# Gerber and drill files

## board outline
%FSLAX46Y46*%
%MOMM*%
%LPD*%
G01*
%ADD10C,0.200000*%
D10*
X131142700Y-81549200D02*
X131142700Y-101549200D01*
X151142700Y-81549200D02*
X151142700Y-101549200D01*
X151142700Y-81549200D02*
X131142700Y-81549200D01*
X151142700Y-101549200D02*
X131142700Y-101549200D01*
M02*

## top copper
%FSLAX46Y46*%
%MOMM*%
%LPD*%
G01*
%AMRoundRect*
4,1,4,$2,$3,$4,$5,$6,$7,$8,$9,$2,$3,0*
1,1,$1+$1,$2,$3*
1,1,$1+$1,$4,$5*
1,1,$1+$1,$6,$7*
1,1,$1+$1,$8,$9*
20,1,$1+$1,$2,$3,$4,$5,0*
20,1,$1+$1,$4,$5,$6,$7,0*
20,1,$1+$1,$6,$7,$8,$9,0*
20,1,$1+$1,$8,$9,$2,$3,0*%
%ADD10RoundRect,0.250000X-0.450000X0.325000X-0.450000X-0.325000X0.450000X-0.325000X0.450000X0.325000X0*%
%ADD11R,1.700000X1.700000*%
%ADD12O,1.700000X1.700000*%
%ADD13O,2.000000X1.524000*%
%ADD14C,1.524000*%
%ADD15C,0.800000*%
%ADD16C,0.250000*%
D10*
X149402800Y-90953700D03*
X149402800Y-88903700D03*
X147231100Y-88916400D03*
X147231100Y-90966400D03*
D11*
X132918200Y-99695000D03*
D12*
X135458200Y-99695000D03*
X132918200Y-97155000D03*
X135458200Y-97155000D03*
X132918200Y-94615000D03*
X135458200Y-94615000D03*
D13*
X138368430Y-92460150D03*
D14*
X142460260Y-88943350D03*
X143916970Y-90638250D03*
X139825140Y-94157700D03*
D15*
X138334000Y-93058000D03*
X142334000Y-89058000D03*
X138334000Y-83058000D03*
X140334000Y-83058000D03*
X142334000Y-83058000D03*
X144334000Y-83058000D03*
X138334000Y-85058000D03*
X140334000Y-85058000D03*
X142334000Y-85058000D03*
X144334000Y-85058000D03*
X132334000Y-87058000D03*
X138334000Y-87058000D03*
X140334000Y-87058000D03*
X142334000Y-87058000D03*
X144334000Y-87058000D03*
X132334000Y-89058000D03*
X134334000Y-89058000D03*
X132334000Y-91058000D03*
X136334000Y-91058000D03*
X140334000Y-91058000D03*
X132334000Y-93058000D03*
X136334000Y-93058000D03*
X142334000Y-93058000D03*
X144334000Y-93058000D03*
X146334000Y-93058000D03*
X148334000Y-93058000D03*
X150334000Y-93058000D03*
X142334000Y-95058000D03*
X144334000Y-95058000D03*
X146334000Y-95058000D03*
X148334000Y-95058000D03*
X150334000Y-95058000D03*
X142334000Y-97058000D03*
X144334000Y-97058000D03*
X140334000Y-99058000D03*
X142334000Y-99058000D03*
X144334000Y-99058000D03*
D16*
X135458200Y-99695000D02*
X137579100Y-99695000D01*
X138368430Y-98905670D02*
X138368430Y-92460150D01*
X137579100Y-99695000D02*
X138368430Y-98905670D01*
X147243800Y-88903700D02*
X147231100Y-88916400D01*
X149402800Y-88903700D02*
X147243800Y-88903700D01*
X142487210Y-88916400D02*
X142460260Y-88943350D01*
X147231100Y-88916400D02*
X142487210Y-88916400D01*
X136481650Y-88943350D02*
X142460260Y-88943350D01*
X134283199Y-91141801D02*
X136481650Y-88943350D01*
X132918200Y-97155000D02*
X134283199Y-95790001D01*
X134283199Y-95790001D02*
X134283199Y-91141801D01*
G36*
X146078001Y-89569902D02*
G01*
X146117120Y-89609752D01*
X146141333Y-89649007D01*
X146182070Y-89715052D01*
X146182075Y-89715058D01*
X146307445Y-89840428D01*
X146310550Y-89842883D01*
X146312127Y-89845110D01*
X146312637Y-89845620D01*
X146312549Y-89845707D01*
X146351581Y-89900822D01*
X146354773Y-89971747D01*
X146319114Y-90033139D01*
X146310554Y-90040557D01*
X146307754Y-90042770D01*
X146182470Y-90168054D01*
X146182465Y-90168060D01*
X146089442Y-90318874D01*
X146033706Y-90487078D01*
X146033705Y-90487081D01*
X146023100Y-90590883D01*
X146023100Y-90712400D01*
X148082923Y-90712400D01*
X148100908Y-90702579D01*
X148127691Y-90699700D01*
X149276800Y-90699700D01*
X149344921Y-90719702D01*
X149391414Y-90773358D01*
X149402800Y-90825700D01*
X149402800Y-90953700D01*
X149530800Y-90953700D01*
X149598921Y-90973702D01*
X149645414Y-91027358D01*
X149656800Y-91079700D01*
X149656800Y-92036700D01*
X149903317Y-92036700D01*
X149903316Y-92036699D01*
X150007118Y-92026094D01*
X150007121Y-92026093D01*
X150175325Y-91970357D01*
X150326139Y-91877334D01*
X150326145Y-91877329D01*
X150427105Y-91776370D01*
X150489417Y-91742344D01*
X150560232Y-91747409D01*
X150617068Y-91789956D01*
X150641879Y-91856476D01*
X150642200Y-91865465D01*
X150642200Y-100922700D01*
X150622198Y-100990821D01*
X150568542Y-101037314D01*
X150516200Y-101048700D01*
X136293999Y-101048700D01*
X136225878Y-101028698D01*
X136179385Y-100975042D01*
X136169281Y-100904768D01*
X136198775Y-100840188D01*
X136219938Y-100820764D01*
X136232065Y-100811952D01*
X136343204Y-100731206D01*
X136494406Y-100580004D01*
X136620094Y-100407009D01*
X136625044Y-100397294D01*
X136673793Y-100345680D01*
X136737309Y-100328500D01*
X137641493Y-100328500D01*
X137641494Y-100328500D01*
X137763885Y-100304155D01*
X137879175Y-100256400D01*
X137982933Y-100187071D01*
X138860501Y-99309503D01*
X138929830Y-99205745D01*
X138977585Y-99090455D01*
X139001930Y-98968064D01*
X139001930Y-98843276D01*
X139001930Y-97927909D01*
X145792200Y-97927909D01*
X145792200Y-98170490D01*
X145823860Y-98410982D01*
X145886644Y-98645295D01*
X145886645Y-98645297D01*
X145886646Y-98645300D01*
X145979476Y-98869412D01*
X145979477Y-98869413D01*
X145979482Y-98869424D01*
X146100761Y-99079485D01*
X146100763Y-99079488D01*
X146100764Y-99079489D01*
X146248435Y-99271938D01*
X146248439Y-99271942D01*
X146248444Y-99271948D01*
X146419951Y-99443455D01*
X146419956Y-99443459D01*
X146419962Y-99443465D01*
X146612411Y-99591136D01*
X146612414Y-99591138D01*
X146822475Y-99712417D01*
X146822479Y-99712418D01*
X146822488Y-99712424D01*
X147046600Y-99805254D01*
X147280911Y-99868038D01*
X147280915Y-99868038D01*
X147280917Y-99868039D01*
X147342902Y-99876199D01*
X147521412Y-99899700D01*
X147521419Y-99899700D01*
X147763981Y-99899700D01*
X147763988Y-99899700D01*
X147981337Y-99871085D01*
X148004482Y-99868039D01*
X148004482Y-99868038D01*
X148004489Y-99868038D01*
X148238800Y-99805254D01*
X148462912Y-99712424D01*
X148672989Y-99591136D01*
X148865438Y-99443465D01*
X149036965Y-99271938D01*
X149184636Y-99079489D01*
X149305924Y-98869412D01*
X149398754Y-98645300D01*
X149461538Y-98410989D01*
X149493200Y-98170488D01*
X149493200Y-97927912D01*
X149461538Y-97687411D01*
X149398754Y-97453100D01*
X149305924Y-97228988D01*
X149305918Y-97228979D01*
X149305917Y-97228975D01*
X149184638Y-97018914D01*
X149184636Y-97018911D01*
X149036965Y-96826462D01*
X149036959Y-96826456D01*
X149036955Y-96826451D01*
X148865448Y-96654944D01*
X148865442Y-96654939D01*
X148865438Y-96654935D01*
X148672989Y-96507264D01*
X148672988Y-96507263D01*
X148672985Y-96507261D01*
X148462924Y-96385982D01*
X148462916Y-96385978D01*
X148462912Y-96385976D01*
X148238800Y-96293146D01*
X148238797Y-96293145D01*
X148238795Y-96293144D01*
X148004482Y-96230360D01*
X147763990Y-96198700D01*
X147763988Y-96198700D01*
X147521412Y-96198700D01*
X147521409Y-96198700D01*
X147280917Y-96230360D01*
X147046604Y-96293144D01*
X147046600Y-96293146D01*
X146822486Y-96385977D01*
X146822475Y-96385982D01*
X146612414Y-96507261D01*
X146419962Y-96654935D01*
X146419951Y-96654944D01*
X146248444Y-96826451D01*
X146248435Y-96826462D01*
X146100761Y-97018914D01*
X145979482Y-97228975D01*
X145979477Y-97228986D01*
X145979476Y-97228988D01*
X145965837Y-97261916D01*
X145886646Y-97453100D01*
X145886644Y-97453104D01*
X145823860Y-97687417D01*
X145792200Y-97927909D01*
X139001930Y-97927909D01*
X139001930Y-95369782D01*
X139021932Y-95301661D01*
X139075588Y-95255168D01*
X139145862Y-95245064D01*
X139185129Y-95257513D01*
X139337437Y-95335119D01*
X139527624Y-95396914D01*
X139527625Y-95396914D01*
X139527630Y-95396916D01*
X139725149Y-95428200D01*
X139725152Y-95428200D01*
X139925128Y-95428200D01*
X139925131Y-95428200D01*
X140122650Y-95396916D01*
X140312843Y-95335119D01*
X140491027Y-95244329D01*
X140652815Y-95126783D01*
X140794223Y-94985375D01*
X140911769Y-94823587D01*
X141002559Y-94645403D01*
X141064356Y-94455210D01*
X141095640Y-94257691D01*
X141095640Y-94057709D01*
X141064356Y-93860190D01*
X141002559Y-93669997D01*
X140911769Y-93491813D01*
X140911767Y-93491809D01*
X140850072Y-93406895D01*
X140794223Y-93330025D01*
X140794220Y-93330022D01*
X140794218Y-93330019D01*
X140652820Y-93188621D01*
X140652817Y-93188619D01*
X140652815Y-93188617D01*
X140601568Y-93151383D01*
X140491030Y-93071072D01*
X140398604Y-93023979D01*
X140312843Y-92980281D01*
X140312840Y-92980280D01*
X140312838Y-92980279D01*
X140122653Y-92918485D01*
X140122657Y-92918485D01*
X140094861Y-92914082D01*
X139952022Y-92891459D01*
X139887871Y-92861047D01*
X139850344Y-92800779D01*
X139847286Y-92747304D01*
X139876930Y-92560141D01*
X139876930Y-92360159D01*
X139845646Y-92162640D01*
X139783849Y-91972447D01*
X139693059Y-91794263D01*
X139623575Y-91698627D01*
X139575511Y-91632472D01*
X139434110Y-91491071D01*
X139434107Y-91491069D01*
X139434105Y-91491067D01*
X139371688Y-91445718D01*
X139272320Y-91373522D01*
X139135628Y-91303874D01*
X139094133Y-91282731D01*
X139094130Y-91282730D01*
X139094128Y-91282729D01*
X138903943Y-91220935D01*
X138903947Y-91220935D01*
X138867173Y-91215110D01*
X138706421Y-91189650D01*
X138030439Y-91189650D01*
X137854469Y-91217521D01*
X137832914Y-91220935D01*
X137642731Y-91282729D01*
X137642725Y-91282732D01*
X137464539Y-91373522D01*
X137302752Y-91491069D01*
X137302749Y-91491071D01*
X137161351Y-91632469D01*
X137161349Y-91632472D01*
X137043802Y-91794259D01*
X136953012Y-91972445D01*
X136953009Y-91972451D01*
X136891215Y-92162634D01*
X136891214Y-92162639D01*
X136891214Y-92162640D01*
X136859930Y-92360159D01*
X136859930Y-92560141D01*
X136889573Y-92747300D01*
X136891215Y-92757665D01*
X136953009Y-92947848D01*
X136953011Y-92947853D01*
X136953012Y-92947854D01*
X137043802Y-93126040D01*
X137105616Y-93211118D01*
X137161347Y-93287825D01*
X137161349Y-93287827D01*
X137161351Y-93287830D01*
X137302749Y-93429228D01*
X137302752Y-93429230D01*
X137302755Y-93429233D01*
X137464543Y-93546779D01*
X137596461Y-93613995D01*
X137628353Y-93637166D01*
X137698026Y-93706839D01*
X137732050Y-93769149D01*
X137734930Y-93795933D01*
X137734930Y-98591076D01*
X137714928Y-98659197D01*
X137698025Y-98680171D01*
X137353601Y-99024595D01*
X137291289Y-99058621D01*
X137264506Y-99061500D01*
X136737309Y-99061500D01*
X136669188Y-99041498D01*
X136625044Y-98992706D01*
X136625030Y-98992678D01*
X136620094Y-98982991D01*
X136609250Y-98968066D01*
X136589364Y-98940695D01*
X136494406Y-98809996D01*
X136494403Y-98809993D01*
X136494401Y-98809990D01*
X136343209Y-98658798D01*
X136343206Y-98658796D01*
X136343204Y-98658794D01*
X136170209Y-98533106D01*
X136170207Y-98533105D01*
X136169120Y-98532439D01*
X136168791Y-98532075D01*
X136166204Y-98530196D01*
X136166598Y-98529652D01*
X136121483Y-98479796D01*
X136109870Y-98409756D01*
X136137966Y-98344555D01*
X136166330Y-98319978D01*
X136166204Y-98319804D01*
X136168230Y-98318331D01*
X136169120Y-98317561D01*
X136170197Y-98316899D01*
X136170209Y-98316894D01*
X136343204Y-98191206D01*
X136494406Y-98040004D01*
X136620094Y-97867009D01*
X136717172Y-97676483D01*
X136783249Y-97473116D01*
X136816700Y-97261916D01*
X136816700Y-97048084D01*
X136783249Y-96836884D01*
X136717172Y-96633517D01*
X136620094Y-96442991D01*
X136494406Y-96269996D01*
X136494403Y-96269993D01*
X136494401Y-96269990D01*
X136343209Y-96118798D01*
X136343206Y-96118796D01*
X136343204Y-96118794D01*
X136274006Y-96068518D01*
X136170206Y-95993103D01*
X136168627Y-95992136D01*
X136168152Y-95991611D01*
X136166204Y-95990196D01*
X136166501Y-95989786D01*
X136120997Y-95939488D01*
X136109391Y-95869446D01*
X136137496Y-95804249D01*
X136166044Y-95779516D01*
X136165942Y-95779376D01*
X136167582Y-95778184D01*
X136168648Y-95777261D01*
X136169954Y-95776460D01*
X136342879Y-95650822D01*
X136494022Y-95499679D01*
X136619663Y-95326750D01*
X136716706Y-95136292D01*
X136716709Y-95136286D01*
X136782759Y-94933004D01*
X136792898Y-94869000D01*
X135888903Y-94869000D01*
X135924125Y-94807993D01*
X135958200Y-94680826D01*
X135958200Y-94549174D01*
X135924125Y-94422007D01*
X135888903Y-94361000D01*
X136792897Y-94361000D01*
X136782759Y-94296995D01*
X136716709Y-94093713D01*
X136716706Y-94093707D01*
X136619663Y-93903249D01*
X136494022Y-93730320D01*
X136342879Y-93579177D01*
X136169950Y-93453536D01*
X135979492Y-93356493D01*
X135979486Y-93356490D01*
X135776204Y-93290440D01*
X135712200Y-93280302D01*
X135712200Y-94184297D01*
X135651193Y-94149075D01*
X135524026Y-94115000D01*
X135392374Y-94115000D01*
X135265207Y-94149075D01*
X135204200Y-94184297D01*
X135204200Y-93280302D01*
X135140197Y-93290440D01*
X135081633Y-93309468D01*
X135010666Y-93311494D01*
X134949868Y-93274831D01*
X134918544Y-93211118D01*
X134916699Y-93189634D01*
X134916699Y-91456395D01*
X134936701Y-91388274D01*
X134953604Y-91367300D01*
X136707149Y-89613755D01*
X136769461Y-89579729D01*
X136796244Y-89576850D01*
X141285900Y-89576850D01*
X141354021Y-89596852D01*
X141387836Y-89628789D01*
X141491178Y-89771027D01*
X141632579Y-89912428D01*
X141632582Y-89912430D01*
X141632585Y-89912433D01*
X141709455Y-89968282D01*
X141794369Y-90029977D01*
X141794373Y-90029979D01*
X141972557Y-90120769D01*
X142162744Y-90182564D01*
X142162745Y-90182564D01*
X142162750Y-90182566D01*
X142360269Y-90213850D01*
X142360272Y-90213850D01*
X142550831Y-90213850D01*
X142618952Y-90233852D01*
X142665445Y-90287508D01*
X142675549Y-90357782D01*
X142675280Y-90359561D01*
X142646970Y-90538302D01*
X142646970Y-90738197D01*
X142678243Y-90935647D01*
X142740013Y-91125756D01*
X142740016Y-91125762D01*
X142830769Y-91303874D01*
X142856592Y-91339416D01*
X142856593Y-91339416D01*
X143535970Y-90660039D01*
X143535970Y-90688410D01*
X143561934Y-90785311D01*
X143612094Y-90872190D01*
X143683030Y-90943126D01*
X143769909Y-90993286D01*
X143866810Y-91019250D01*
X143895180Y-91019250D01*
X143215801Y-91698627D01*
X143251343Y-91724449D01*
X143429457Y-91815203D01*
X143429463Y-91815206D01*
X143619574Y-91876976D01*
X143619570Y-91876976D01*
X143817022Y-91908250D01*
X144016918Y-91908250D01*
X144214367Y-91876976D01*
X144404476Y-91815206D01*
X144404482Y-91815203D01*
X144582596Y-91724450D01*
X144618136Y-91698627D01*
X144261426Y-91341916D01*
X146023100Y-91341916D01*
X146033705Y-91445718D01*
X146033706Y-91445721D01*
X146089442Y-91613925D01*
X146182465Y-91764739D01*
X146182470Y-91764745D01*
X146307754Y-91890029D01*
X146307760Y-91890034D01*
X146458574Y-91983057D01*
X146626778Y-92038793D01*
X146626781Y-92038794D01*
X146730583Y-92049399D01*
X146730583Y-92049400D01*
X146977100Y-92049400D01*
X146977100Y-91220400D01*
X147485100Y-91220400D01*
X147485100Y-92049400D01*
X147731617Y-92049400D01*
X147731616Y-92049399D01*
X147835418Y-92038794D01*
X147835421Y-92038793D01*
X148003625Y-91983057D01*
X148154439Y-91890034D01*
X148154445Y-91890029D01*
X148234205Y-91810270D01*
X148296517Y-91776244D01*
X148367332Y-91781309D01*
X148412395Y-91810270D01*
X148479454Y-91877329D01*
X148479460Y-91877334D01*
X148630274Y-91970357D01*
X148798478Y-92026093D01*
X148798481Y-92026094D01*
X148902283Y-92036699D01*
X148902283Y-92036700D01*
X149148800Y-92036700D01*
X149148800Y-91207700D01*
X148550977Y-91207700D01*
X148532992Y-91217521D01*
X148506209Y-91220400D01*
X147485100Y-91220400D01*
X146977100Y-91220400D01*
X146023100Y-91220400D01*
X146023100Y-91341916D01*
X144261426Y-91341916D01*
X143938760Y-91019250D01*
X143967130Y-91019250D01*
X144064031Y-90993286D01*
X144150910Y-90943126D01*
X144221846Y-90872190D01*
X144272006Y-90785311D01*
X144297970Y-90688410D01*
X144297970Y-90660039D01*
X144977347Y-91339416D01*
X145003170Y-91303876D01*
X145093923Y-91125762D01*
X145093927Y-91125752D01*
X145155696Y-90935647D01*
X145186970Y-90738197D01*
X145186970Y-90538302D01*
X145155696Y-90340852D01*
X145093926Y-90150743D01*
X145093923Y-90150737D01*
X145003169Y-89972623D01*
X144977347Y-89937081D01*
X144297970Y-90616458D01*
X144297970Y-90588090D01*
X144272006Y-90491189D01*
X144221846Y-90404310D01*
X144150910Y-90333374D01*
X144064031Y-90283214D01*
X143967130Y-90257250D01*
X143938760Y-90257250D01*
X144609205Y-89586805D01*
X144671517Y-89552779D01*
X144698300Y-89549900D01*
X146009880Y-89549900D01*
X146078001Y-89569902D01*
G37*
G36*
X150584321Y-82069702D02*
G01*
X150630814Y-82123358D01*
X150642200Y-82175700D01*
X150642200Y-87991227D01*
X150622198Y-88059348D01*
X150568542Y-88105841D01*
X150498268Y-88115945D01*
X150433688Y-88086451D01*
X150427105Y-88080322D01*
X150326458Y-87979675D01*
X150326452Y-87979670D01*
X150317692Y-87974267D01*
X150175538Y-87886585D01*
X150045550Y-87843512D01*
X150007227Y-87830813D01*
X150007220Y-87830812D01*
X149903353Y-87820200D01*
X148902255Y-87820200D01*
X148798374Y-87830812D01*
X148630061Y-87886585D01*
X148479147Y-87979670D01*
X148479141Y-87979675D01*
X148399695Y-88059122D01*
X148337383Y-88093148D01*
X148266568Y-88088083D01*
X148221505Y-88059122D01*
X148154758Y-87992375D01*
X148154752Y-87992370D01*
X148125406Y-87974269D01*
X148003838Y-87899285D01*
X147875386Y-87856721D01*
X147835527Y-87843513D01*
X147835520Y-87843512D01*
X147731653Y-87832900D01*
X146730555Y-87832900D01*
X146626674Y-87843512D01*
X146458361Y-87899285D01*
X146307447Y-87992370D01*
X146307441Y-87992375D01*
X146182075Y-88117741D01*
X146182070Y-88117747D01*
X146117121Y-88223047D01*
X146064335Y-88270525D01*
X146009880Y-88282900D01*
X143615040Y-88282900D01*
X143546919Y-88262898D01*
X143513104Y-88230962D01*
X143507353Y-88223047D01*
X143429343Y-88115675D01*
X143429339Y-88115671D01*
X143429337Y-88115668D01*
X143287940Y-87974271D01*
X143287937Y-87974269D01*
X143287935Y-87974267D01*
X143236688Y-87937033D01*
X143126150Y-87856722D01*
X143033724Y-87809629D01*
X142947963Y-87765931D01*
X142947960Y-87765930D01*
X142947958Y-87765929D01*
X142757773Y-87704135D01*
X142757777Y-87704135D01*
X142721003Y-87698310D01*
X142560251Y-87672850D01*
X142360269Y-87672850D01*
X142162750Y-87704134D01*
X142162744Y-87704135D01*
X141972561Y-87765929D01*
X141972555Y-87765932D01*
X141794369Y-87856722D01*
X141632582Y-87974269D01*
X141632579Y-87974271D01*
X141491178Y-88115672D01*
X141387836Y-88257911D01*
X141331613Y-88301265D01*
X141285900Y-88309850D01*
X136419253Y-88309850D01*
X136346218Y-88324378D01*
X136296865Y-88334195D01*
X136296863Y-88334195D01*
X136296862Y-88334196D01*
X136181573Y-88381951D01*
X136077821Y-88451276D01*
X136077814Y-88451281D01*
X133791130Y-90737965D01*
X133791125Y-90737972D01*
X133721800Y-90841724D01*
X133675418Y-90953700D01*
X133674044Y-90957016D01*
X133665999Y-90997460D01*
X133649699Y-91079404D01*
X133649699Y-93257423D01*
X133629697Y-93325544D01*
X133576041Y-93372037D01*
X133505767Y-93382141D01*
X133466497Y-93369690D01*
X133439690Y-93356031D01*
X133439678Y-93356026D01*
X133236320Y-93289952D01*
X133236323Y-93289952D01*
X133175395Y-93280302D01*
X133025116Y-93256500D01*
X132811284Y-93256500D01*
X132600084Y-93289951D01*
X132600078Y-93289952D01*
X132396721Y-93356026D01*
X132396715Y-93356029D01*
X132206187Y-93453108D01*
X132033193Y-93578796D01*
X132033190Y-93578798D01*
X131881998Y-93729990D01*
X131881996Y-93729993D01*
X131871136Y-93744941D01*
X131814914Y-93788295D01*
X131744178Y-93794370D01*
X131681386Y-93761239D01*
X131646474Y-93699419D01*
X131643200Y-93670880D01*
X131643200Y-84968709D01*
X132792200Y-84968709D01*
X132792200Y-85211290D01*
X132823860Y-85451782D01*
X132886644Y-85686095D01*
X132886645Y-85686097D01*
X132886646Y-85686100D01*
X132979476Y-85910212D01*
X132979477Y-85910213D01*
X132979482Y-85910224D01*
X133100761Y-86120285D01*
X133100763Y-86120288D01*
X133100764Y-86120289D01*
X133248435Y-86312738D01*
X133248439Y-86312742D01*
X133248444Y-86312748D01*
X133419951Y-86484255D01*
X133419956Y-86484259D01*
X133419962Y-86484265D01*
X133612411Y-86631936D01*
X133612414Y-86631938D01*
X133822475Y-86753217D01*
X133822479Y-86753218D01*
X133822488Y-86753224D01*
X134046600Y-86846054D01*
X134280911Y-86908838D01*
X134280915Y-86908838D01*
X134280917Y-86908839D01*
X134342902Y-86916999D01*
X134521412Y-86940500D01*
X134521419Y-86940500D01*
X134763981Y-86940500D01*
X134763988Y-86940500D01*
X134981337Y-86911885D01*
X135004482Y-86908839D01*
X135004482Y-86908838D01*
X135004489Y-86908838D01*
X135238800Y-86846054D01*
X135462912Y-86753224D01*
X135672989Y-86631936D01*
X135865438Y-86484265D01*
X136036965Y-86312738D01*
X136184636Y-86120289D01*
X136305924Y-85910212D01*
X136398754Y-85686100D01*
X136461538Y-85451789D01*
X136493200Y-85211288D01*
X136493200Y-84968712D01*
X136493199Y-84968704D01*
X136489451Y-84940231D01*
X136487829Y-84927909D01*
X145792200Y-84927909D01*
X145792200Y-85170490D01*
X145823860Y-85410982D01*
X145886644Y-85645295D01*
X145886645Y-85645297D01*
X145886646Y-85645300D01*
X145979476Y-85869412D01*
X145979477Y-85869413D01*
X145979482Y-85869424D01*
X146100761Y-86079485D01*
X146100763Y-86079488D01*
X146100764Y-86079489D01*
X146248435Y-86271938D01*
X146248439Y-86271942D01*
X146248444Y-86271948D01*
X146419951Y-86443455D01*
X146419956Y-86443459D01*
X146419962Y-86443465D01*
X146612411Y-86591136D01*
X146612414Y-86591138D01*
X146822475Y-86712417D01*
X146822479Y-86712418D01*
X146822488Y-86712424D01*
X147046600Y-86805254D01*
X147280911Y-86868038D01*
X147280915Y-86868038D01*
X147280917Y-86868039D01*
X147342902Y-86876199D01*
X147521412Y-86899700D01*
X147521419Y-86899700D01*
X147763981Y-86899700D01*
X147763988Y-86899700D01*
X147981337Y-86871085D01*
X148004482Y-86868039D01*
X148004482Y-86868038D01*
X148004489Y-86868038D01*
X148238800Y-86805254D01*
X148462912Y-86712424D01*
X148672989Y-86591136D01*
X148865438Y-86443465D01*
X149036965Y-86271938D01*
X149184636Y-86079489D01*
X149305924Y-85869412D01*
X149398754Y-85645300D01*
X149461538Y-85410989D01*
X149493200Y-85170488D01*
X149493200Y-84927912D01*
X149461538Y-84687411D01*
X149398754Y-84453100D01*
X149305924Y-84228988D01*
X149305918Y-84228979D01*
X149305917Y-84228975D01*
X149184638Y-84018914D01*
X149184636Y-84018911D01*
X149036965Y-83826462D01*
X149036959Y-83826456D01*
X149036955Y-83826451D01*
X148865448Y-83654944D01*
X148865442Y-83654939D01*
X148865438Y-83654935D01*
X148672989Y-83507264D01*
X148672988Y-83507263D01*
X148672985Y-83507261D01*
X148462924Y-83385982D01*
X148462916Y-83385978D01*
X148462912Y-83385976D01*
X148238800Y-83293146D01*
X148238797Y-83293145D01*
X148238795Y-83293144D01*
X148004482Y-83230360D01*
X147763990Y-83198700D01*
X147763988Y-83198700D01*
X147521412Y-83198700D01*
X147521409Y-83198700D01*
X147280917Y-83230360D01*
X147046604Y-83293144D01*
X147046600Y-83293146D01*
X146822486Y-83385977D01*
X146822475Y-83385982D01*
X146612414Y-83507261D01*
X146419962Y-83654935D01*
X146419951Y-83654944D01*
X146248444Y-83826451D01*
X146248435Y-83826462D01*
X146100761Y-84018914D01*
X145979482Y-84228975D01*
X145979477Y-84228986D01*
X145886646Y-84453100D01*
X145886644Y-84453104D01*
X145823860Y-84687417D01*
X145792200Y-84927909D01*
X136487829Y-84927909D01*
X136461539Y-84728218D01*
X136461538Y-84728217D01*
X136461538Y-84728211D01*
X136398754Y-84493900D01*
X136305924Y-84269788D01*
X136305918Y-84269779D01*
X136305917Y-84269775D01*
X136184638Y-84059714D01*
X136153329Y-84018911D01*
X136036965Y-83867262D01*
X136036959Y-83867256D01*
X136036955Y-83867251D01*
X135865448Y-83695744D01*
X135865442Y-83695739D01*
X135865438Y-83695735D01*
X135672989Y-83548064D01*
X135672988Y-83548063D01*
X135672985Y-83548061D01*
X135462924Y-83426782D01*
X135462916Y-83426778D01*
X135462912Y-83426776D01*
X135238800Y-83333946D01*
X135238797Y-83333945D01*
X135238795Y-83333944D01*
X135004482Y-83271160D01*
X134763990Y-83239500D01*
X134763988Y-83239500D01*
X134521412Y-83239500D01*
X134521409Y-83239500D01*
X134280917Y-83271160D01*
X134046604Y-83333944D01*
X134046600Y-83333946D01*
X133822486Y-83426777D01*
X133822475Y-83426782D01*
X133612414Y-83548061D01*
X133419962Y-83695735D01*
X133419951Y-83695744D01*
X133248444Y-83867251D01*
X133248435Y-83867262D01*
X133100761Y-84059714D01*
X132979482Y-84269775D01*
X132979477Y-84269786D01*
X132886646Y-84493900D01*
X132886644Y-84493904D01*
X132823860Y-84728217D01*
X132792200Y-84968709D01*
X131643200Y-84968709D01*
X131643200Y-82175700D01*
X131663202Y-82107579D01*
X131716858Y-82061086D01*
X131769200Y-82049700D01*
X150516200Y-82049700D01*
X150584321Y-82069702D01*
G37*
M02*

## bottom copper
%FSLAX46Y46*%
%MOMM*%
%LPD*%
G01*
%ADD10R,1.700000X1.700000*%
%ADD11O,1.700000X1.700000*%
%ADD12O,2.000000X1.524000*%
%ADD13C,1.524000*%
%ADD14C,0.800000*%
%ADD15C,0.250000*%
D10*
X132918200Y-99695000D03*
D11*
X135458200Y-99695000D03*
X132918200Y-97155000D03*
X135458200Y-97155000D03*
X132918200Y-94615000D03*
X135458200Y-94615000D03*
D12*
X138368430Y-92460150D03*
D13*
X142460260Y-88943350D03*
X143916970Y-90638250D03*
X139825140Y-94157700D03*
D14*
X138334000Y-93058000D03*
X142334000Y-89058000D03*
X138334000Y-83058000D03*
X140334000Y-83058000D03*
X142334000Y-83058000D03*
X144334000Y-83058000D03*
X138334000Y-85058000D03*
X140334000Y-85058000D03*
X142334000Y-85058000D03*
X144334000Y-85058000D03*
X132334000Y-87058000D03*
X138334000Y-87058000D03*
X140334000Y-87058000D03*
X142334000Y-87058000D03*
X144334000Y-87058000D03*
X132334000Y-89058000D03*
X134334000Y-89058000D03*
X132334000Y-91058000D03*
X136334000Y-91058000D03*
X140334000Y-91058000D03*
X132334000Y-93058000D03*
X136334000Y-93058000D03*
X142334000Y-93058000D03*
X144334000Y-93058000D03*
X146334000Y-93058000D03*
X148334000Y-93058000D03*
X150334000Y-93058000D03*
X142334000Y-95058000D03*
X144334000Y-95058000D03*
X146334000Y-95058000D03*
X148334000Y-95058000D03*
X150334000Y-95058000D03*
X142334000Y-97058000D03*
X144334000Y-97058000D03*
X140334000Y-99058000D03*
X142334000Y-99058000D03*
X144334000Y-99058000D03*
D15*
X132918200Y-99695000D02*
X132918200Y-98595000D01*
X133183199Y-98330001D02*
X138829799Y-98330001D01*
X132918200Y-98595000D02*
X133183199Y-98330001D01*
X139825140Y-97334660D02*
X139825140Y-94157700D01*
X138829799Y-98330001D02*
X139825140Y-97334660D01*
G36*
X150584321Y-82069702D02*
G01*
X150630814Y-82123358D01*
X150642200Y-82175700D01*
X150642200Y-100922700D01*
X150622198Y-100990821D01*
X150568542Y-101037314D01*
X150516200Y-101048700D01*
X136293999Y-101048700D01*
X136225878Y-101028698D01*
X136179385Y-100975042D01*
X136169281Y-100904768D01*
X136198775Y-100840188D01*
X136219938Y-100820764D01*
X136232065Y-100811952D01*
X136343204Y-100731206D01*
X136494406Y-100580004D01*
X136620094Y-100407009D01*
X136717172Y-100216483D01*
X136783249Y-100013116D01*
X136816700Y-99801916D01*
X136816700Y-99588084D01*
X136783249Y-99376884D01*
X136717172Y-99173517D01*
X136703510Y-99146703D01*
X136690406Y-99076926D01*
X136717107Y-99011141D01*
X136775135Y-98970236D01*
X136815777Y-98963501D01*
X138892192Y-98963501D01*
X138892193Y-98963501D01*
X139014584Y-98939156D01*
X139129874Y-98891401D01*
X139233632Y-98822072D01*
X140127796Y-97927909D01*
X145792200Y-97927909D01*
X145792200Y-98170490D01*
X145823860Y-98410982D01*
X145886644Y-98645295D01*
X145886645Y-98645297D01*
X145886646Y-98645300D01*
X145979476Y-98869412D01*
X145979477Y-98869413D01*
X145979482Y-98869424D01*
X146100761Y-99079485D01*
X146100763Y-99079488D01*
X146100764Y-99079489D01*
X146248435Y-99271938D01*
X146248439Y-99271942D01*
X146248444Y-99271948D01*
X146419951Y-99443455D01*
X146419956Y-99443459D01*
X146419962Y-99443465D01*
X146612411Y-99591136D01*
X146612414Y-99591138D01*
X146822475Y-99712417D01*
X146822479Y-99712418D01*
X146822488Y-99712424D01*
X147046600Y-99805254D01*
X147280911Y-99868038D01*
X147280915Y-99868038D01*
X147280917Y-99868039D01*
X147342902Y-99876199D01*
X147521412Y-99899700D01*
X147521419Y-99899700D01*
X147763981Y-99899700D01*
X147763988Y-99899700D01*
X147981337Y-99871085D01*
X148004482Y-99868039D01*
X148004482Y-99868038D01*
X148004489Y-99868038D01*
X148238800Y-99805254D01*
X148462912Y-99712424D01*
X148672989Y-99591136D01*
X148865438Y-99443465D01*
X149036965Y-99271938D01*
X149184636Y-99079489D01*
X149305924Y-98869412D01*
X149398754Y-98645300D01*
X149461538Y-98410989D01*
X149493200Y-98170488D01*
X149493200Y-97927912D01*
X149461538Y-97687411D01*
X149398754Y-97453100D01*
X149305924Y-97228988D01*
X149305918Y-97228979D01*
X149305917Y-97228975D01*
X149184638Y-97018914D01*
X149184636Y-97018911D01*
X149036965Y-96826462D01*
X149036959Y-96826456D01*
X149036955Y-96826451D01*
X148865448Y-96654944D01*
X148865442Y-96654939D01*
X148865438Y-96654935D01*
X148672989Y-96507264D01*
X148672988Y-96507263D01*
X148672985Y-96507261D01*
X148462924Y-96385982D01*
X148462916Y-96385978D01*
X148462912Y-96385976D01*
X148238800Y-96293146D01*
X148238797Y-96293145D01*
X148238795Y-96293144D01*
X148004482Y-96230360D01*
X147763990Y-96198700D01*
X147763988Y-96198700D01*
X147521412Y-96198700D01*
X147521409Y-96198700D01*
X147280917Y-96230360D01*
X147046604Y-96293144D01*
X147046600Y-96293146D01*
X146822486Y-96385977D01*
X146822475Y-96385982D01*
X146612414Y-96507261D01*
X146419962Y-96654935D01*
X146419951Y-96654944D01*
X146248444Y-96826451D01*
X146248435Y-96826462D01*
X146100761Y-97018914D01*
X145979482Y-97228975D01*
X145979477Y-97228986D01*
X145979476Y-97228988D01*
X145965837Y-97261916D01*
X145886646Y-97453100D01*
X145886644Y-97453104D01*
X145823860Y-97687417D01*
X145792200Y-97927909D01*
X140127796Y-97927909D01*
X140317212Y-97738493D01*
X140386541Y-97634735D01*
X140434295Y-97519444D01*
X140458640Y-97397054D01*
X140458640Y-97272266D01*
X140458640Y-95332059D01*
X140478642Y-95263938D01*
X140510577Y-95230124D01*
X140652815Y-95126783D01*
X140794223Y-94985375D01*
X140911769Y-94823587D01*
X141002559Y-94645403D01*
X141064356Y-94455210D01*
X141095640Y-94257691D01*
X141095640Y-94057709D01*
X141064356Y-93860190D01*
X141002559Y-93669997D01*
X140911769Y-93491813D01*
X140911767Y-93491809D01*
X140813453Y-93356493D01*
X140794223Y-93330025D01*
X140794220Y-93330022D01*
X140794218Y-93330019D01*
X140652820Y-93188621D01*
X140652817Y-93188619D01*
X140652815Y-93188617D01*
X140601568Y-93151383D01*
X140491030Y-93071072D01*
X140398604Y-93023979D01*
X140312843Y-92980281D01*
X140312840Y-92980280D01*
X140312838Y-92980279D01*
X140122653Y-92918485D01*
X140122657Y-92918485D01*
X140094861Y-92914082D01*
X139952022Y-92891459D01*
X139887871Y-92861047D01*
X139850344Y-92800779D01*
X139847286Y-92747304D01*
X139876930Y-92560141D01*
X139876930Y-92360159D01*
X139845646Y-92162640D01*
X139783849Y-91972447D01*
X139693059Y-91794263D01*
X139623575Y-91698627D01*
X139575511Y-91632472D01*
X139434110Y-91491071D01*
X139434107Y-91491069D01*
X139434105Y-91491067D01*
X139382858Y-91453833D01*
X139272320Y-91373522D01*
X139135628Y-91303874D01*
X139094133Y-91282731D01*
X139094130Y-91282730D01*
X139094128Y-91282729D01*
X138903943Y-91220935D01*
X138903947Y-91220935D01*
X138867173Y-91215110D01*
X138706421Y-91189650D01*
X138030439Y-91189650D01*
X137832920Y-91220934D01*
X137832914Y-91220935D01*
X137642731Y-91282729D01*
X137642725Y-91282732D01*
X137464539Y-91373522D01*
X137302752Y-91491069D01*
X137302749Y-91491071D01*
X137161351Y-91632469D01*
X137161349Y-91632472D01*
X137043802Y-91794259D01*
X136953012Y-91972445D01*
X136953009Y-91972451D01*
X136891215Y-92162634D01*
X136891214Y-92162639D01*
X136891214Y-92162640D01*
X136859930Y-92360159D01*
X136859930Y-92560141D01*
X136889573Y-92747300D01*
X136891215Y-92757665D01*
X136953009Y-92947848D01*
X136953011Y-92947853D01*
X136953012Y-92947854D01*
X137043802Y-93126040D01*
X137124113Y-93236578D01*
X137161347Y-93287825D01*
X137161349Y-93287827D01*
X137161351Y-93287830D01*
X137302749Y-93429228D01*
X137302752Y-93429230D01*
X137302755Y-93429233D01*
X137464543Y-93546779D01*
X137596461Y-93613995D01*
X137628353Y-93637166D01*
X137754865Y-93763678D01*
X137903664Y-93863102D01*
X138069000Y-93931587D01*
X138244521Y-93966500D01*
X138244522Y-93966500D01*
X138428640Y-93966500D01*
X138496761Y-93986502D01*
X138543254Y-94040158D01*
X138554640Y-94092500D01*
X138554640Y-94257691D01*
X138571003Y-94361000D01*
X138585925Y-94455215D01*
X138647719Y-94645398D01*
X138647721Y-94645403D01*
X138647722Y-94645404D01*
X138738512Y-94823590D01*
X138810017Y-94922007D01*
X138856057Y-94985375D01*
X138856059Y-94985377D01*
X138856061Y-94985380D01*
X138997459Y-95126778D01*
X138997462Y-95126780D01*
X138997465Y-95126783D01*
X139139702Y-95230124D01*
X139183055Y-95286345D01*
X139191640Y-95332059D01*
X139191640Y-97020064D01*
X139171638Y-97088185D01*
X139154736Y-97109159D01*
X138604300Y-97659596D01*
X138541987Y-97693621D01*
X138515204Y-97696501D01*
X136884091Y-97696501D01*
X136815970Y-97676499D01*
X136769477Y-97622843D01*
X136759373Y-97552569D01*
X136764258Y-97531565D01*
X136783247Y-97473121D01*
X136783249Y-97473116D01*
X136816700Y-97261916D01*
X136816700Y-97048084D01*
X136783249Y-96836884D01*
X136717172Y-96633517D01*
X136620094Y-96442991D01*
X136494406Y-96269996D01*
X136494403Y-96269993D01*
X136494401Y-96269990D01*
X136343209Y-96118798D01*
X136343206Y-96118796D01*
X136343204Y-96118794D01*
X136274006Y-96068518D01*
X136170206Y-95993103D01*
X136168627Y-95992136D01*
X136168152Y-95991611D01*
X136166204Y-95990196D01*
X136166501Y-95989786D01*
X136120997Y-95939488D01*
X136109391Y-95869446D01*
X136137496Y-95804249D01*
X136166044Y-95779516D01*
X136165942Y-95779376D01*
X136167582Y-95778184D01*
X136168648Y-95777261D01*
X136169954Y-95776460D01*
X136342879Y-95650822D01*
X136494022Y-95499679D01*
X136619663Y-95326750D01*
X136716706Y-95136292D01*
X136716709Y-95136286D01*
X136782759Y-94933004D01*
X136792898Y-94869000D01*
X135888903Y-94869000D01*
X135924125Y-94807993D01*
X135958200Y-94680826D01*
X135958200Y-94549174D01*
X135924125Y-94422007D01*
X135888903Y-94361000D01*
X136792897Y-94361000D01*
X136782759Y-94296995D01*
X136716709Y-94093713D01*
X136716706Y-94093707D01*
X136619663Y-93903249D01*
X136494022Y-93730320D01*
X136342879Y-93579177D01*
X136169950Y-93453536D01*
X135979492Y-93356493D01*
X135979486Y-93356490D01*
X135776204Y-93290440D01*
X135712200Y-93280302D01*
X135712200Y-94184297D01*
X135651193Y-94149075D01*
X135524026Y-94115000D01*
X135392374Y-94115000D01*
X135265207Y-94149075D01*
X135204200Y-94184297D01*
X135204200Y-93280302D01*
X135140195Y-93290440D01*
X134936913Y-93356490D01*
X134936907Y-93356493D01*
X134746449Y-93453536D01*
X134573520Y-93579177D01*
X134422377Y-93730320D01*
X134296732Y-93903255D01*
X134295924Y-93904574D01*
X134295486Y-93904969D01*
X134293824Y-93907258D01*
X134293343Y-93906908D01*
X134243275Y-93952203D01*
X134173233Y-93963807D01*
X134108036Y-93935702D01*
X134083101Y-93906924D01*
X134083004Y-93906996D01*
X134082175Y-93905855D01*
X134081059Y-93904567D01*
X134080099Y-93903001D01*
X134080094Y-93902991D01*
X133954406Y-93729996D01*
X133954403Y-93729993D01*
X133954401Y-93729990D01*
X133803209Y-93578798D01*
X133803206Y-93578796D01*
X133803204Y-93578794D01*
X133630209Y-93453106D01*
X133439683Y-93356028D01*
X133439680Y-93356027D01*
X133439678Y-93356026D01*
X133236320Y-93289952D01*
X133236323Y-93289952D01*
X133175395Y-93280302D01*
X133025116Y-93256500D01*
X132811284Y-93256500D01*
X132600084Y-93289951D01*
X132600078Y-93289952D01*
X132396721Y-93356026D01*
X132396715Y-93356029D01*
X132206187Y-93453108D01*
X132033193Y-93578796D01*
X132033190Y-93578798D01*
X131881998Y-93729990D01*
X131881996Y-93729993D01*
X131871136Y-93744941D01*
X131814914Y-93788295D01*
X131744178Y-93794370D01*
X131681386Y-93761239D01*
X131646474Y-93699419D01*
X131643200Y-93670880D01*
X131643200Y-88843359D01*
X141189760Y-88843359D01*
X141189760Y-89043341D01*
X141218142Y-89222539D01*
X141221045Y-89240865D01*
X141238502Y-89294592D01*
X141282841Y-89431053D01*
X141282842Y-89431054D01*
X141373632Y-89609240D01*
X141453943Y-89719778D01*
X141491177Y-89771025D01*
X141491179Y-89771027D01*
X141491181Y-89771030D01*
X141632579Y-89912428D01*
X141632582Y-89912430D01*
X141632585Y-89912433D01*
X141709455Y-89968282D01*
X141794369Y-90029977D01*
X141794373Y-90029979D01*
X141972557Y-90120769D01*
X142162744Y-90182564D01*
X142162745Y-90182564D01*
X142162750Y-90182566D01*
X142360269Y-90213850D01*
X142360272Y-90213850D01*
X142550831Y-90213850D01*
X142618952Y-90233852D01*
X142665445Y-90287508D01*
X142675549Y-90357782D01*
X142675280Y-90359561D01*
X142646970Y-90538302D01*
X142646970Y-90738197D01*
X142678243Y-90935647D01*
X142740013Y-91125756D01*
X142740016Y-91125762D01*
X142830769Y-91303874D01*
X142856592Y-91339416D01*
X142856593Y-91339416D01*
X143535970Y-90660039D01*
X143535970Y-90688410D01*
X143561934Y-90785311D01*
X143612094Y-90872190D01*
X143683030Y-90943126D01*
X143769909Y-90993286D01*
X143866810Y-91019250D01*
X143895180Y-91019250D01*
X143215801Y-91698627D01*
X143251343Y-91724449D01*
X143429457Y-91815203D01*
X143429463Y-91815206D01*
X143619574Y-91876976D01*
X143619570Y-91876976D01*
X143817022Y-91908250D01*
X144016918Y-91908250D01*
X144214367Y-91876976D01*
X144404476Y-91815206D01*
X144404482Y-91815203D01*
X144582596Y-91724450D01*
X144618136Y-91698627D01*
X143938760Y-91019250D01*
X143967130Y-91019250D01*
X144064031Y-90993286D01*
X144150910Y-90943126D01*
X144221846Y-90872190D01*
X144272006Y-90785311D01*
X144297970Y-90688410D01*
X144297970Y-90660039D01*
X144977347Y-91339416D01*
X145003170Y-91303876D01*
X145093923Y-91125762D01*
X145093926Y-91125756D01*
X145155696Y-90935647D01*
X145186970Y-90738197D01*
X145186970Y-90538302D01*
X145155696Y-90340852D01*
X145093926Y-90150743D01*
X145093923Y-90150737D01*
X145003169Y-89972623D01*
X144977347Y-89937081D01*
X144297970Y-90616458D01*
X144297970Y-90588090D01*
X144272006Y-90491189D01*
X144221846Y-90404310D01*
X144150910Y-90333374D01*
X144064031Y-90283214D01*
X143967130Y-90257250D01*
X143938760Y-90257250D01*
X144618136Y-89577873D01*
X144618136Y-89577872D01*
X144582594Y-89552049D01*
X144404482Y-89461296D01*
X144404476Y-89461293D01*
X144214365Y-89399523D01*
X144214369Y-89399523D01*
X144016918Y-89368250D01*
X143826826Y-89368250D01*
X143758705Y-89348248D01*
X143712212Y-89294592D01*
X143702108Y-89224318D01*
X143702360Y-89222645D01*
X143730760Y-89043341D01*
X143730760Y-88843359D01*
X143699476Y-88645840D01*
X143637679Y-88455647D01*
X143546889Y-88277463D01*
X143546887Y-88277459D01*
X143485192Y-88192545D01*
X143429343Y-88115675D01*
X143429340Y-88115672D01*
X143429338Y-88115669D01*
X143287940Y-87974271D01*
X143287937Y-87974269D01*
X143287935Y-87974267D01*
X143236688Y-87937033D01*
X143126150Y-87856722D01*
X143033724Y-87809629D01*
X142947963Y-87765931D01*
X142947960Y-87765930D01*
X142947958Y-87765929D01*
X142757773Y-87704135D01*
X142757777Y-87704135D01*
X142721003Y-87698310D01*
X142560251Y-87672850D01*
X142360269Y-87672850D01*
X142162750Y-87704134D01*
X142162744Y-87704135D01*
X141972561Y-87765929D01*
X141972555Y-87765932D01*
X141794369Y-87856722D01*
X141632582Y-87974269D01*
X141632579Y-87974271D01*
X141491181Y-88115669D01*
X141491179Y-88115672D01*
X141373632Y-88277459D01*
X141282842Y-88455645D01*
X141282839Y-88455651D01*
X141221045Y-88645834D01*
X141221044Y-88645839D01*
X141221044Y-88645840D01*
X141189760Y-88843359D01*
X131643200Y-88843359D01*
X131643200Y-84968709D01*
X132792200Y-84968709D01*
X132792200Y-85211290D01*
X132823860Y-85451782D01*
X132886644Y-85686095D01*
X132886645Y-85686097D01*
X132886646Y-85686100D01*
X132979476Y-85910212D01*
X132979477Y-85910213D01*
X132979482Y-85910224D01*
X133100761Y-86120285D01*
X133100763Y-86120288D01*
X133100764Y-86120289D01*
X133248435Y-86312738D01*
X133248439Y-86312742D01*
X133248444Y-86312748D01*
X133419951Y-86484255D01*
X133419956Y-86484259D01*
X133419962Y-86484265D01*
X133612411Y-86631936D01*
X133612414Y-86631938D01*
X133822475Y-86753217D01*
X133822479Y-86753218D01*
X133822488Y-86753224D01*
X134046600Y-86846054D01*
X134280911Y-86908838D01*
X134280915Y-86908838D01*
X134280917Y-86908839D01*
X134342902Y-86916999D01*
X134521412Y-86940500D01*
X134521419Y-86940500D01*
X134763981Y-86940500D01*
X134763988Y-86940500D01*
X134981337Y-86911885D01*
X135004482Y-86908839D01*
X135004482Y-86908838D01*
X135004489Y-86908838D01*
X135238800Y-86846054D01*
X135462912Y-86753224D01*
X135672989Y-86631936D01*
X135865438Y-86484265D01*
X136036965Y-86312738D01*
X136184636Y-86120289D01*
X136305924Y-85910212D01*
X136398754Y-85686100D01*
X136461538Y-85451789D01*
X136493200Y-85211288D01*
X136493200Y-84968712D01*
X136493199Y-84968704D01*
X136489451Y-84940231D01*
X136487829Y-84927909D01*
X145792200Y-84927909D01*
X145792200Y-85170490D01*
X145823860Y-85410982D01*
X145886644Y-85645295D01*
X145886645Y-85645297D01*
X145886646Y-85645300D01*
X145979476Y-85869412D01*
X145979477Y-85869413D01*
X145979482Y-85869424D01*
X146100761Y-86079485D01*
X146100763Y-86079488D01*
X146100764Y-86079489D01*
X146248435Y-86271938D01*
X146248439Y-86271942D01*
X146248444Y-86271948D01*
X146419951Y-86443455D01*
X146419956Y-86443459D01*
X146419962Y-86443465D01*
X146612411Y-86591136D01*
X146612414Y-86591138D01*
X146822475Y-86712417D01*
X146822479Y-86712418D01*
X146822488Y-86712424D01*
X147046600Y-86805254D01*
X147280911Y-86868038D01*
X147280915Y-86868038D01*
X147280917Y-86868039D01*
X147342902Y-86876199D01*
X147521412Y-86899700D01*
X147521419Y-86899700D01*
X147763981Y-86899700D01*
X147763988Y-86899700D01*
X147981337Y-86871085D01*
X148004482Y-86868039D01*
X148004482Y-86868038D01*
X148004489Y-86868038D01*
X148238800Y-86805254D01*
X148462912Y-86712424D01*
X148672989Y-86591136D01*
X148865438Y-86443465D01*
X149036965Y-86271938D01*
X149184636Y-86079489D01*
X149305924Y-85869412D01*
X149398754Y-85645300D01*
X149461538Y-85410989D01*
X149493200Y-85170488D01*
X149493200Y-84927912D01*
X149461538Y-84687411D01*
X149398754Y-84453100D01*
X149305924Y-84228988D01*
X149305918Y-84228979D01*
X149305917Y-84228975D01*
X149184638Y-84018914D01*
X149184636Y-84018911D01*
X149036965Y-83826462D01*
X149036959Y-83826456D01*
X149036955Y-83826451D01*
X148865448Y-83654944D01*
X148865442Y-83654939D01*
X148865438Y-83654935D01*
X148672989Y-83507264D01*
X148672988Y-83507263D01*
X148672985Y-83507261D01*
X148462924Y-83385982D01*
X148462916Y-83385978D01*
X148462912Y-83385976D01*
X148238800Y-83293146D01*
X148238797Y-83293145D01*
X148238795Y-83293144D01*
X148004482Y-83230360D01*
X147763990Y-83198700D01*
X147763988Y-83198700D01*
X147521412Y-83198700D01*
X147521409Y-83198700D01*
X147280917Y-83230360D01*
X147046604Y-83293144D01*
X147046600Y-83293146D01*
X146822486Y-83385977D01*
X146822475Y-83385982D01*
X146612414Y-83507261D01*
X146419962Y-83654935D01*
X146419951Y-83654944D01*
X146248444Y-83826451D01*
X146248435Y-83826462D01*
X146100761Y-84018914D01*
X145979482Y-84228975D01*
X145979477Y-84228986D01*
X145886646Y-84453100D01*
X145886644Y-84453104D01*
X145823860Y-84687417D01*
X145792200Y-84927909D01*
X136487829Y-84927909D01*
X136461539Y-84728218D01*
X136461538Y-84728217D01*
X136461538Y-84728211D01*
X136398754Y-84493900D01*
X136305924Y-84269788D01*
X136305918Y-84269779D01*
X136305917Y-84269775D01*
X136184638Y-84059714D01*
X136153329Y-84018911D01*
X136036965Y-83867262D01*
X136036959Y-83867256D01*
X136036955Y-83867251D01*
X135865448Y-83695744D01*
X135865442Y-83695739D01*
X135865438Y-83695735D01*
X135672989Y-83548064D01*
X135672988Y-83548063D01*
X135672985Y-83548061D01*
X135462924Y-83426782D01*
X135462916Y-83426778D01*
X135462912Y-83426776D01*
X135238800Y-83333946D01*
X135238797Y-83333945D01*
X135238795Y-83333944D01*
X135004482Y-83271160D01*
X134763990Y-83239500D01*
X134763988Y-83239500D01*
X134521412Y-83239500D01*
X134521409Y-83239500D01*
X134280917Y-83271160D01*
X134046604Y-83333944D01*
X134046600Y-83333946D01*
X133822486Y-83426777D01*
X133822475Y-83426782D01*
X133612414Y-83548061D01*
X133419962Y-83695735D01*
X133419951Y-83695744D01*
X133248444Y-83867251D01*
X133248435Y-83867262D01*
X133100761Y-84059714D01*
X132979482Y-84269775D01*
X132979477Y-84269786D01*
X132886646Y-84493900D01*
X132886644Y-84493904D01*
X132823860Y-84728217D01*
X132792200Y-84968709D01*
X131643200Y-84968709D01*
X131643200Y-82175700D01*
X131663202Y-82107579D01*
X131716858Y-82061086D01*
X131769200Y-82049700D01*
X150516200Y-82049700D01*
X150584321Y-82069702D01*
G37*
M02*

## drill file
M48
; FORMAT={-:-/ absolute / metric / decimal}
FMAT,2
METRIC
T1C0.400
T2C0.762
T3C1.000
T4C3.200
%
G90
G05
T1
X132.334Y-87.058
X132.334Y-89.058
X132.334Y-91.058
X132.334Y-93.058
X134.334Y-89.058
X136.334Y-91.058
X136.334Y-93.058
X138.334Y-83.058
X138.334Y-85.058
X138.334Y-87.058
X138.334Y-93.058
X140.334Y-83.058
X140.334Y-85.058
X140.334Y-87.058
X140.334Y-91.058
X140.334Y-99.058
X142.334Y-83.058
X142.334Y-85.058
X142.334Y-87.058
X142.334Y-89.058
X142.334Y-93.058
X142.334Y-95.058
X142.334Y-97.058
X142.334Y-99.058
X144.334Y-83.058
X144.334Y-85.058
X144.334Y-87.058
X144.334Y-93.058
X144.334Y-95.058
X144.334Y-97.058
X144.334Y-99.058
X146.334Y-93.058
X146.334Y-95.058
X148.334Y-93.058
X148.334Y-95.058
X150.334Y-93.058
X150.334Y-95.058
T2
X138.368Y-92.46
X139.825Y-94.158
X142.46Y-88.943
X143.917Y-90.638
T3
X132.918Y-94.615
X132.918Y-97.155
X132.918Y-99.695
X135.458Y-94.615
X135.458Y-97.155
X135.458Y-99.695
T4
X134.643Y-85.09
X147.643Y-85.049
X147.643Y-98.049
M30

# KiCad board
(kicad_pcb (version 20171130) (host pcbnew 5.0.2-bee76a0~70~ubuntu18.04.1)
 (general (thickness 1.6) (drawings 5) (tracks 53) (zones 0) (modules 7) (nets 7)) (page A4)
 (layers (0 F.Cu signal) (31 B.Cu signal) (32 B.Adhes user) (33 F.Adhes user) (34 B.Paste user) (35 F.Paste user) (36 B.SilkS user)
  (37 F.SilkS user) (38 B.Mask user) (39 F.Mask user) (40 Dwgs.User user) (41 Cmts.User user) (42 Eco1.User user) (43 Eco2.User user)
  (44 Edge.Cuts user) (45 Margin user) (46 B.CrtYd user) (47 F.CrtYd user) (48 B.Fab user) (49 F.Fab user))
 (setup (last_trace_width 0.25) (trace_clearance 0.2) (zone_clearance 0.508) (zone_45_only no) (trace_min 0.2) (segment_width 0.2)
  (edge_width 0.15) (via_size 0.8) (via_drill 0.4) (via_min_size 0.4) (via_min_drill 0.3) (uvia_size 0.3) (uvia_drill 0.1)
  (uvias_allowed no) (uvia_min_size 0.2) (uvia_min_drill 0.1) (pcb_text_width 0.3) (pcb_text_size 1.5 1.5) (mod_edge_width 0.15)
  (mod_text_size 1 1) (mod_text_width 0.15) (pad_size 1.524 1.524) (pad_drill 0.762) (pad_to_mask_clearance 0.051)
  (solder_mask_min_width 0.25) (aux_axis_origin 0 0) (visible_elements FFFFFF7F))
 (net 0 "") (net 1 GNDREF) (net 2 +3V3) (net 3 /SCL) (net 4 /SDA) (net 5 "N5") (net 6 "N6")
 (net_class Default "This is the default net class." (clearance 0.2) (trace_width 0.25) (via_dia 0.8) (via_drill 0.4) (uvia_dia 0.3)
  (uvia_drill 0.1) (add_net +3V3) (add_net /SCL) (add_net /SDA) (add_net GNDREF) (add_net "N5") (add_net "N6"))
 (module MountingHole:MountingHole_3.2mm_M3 (layer F.Cu) (at 134.6427 85.09)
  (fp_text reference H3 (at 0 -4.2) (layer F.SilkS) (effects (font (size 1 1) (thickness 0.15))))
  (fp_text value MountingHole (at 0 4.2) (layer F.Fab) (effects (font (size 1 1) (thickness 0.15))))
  (pad 1 np_thru_hole circle (at 0 0) (size 3.2 3.2) (drill 3.2) (layers *.Cu *.Mask)))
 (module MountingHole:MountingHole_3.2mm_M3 (layer F.Cu) (at 147.6427 85.0492)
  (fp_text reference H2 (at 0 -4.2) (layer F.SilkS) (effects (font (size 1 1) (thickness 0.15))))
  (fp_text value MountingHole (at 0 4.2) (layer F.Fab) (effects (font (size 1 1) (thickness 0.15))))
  (pad 1 np_thru_hole circle (at 0 0) (size 3.2 3.2) (drill 3.2) (layers *.Cu *.Mask)))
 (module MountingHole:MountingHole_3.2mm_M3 (layer F.Cu) (at 147.6427 98.0492)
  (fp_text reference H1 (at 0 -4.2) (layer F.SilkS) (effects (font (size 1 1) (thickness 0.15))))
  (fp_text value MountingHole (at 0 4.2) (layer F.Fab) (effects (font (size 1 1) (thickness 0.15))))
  (pad 1 np_thru_hole circle (at 0 0) (size 3.2 3.2) (drill 3.2) (layers *.Cu *.Mask)))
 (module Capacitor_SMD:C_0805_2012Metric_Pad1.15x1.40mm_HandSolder (layer F.Cu) (at 149.4028 89.9287 270)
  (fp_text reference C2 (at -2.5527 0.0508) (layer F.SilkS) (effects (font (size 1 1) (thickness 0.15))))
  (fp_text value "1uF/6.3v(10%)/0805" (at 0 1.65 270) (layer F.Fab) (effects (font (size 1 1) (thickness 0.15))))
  (pad 2 smd roundrect (at 1.025 0 270) (size 1.15 1.4) (layers F.Cu F.Paste F.Mask) (roundrect_rratio 0.217391) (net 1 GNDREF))
  (pad 1 smd roundrect (at -1.025 0 270) (size 1.15 1.4) (layers F.Cu F.Paste F.Mask) (roundrect_rratio 0.217391) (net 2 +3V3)))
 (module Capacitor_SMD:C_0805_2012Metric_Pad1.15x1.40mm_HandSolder (layer F.Cu) (at 147.2311 89.9414 270)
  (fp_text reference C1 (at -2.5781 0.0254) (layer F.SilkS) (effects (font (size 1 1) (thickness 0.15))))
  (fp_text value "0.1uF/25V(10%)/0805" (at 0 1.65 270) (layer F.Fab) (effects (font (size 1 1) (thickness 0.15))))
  (pad 1 smd roundrect (at -1.025 0 270) (size 1.15 1.4) (layers F.Cu F.Paste F.Mask) (roundrect_rratio 0.217391) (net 2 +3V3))
  (pad 2 smd roundrect (at 1.025 0 270) (size 1.15 1.4) (layers F.Cu F.Paste F.Mask) (roundrect_rratio 0.217391) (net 1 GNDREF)))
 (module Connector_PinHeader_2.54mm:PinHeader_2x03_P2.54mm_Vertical (layer B.Cu) (at 132.9182 99.695)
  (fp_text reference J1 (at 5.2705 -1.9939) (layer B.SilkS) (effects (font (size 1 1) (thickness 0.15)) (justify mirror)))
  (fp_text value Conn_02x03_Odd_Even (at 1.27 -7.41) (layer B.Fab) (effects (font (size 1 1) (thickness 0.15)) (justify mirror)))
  (pad 1 thru_hole rect (at 0 0) (size 1.7 1.7) (drill 1) (layers *.Cu *.Mask) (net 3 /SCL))
  (pad 2 thru_hole oval (at 2.54 0) (size 1.7 1.7) (drill 1) (layers *.Cu *.Mask) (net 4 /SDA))
  (pad 3 thru_hole oval (at 0 -2.54) (size 1.7 1.7) (drill 1) (layers *.Cu *.Mask) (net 2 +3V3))
  (pad 4 thru_hole oval (at 2.54 -2.54) (size 1.7 1.7) (drill 1) (layers *.Cu *.Mask) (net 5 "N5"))
  (pad 5 thru_hole oval (at 0 -5.08) (size 1.7 1.7) (drill 1) (layers *.Cu *.Mask) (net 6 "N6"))
  (pad 6 thru_hole oval (at 2.54 -5.08) (size 1.7 1.7) (drill 1) (layers *.Cu *.Mask) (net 1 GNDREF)))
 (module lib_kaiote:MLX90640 (layer F.Cu) (at 141.1427 91.5492)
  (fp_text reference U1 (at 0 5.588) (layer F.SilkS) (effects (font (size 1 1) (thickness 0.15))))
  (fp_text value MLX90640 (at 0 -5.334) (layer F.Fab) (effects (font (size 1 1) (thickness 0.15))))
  (pad 1 thru_hole oval (at -2.77427 0.91095) (size 2 1.524) (drill 0.762) (layers *.Cu *.Mask) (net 4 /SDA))
  (pad 2 thru_hole circle (at 1.31756 -2.60585) (size 1.524 1.524) (drill 0.762) (layers *.Cu *.Mask) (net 2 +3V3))
  (pad 3 thru_hole circle (at 2.77427 -0.91095) (size 1.524 1.524) (drill 0.762) (layers *.Cu *.Mask) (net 1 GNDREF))
  (pad 4 thru_hole circle (at -1.31756 2.6085) (size 1.524 1.524) (drill 0.762) (layers *.Cu *.Mask) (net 3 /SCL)))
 (gr_line (start 131.1427 81.5492) (end 131.1427 101.5492) (layer Edge.Cuts) (width 0.2))
 (gr_line (start 151.1427 81.5492) (end 151.1427 101.5492) (layer Edge.Cuts) (width 0.2))
 (gr_line (start 151.1427 81.5492) (end 131.1427 81.5492) (layer Edge.Cuts) (width 0.2))
 (gr_line (start 151.1427 101.5492) (end 131.1427 101.5492) (layer Edge.Cuts) (width 0.2))
 (segment (start 135.4582 99.695) (end 137.5791 99.695) (width 0.25) (layer F.Cu) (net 4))
 (segment (start 138.36843 98.90567) (end 138.36843 92.46015) (width 0.25) (layer F.Cu) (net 4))
 (segment (start 137.5791 99.695) (end 138.36843 98.90567) (width 0.25) (layer F.Cu) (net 4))
 (via (at 138.334 93.058) (size 0.8) (drill 0.4) (layers F.Cu B.Cu) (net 4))
 (segment (start 147.2438 88.9037) (end 147.2311 88.9164) (width 0.25) (layer F.Cu) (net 2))
 (segment (start 149.4028 88.9037) (end 147.2438 88.9037) (width 0.25) (layer F.Cu) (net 2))
 (segment (start 142.48721 88.9164) (end 142.46026 88.94335) (width 0.25) (layer F.Cu) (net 2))
 (segment (start 147.2311 88.9164) (end 142.48721 88.9164) (width 0.25) (layer F.Cu) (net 2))
 (segment (start 136.48165 88.94335) (end 142.46026 88.94335) (width 0.25) (layer F.Cu) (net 2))
 (segment (start 134.283199 91.141801) (end 136.48165 88.94335) (width 0.25) (layer F.Cu) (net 2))
 (segment (start 132.9182 97.155) (end 134.283199 95.790001) (width 0.25) (layer F.Cu) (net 2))
 (segment (start 134.283199 95.790001) (end 134.283199 91.141801) (width 0.25) (layer F.Cu) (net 2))
 (via (at 142.334 89.058) (size 0.8) (drill 0.4) (layers F.Cu B.Cu) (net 2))
 (via (at 138.334 83.058) (size 0.8) (drill 0.4) (layers F.Cu B.Cu) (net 1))
 (via (at 140.334 83.058) (size 0.8) (drill 0.4) (layers F.Cu B.Cu) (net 1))
 (via (at 142.334 83.058) (size 0.8) (drill 0.4) (layers F.Cu B.Cu) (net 1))
 (via (at 144.334 83.058) (size 0.8) (drill 0.4) (layers F.Cu B.Cu) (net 1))
 (via (at 138.334 85.058) (size 0.8) (drill 0.4) (layers F.Cu B.Cu) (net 1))
 (via (at 140.334 85.058) (size 0.8) (drill 0.4) (layers F.Cu B.Cu) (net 1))
 (via (at 142.334 85.058) (size 0.8) (drill 0.4) (layers F.Cu B.Cu) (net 1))
 (via (at 144.334 85.058) (size 0.8) (drill 0.4) (layers F.Cu B.Cu) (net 1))
 (via (at 132.334 87.058) (size 0.8) (drill 0.4) (layers F.Cu B.Cu) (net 1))
 (via (at 138.334 87.058) (size 0.8) (drill 0.4) (layers F.Cu B.Cu) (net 1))
 (via (at 140.334 87.058) (size 0.8) (drill 0.4) (layers F.Cu B.Cu) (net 1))
 (via (at 142.334 87.058) (size 0.8) (drill 0.4) (layers F.Cu B.Cu) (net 1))
 (via (at 144.334 87.058) (size 0.8) (drill 0.4) (layers F.Cu B.Cu) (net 1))
 (via (at 132.334 89.058) (size 0.8) (drill 0.4) (layers F.Cu B.Cu) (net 1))
 (via (at 134.334 89.058) (size 0.8) (drill 0.4) (layers F.Cu B.Cu) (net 1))
 (via (at 132.334 91.058) (size 0.8) (drill 0.4) (layers F.Cu B.Cu) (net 1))
 (via (at 136.334 91.058) (size 0.8) (drill 0.4) (layers F.Cu B.Cu) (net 1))
 (via (at 140.334 91.058) (size 0.8) (drill 0.4) (layers F.Cu B.Cu) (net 1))
 (via (at 132.334 93.058) (size 0.8) (drill 0.4) (layers F.Cu B.Cu) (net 1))
 (via (at 136.334 93.058) (size 0.8) (drill 0.4) (layers F.Cu B.Cu) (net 1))
 (via (at 142.334 93.058) (size 0.8) (drill 0.4) (layers F.Cu B.Cu) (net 1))
 (via (at 144.334 93.058) (size 0.8) (drill 0.4) (layers F.Cu B.Cu) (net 1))
 (via (at 146.334 93.058) (size 0.8) (drill 0.4) (layers F.Cu B.Cu) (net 1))
 (via (at 148.334 93.058) (size 0.8) (drill 0.4) (layers F.Cu B.Cu) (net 1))
 (via (at 150.334 93.058) (size 0.8) (drill 0.4) (layers F.Cu B.Cu) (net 1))
 (via (at 142.334 95.058) (size 0.8) (drill 0.4) (layers F.Cu B.Cu) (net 1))
 (via (at 144.334 95.058) (size 0.8) (drill 0.4) (layers F.Cu B.Cu) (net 1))
 (via (at 146.334 95.058) (size 0.8) (drill 0.4) (layers F.Cu B.Cu) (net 1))
 (via (at 148.334 95.058) (size 0.8) (drill 0.4) (layers F.Cu B.Cu) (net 1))
 (via (at 150.334 95.058) (size 0.8) (drill 0.4) (layers F.Cu B.Cu) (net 1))
 (via (at 142.334 97.058) (size 0.8) (drill 0.4) (layers F.Cu B.Cu) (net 1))
 (via (at 144.334 97.058) (size 0.8) (drill 0.4) (layers F.Cu B.Cu) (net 1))
 (via (at 140.334 99.058) (size 0.8) (drill 0.4) (layers F.Cu B.Cu) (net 1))
 (via (at 142.334 99.058) (size 0.8) (drill 0.4) (layers F.Cu B.Cu) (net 1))
 (via (at 144.334 99.058) (size 0.8) (drill 0.4) (layers F.Cu B.Cu) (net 1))
 (segment (start 132.9182 99.695) (end 132.9182 98.595) (width 0.25) (layer B.Cu) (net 3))
 (segment (start 133.183199 98.330001) (end 138.829799 98.330001) (width 0.25) (layer B.Cu) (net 3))
 (segment (start 132.9182 98.595) (end 133.183199 98.330001) (width 0.25) (layer B.Cu) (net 3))
 (segment (start 139.82514 97.33466) (end 139.82514 94.1577) (width 0.25) (layer B.Cu) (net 3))
 (segment (start 138.829799 98.330001) (end 139.82514 97.33466) (width 0.25) (layer B.Cu) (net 3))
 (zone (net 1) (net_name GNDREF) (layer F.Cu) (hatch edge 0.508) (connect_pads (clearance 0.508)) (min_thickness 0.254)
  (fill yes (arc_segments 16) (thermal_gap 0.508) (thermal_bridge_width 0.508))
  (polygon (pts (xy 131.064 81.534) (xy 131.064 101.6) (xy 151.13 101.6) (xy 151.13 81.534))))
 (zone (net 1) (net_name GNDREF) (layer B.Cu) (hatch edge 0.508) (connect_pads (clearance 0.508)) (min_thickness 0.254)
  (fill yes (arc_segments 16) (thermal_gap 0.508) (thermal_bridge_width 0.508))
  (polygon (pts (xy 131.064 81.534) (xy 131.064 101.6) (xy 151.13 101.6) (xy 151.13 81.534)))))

